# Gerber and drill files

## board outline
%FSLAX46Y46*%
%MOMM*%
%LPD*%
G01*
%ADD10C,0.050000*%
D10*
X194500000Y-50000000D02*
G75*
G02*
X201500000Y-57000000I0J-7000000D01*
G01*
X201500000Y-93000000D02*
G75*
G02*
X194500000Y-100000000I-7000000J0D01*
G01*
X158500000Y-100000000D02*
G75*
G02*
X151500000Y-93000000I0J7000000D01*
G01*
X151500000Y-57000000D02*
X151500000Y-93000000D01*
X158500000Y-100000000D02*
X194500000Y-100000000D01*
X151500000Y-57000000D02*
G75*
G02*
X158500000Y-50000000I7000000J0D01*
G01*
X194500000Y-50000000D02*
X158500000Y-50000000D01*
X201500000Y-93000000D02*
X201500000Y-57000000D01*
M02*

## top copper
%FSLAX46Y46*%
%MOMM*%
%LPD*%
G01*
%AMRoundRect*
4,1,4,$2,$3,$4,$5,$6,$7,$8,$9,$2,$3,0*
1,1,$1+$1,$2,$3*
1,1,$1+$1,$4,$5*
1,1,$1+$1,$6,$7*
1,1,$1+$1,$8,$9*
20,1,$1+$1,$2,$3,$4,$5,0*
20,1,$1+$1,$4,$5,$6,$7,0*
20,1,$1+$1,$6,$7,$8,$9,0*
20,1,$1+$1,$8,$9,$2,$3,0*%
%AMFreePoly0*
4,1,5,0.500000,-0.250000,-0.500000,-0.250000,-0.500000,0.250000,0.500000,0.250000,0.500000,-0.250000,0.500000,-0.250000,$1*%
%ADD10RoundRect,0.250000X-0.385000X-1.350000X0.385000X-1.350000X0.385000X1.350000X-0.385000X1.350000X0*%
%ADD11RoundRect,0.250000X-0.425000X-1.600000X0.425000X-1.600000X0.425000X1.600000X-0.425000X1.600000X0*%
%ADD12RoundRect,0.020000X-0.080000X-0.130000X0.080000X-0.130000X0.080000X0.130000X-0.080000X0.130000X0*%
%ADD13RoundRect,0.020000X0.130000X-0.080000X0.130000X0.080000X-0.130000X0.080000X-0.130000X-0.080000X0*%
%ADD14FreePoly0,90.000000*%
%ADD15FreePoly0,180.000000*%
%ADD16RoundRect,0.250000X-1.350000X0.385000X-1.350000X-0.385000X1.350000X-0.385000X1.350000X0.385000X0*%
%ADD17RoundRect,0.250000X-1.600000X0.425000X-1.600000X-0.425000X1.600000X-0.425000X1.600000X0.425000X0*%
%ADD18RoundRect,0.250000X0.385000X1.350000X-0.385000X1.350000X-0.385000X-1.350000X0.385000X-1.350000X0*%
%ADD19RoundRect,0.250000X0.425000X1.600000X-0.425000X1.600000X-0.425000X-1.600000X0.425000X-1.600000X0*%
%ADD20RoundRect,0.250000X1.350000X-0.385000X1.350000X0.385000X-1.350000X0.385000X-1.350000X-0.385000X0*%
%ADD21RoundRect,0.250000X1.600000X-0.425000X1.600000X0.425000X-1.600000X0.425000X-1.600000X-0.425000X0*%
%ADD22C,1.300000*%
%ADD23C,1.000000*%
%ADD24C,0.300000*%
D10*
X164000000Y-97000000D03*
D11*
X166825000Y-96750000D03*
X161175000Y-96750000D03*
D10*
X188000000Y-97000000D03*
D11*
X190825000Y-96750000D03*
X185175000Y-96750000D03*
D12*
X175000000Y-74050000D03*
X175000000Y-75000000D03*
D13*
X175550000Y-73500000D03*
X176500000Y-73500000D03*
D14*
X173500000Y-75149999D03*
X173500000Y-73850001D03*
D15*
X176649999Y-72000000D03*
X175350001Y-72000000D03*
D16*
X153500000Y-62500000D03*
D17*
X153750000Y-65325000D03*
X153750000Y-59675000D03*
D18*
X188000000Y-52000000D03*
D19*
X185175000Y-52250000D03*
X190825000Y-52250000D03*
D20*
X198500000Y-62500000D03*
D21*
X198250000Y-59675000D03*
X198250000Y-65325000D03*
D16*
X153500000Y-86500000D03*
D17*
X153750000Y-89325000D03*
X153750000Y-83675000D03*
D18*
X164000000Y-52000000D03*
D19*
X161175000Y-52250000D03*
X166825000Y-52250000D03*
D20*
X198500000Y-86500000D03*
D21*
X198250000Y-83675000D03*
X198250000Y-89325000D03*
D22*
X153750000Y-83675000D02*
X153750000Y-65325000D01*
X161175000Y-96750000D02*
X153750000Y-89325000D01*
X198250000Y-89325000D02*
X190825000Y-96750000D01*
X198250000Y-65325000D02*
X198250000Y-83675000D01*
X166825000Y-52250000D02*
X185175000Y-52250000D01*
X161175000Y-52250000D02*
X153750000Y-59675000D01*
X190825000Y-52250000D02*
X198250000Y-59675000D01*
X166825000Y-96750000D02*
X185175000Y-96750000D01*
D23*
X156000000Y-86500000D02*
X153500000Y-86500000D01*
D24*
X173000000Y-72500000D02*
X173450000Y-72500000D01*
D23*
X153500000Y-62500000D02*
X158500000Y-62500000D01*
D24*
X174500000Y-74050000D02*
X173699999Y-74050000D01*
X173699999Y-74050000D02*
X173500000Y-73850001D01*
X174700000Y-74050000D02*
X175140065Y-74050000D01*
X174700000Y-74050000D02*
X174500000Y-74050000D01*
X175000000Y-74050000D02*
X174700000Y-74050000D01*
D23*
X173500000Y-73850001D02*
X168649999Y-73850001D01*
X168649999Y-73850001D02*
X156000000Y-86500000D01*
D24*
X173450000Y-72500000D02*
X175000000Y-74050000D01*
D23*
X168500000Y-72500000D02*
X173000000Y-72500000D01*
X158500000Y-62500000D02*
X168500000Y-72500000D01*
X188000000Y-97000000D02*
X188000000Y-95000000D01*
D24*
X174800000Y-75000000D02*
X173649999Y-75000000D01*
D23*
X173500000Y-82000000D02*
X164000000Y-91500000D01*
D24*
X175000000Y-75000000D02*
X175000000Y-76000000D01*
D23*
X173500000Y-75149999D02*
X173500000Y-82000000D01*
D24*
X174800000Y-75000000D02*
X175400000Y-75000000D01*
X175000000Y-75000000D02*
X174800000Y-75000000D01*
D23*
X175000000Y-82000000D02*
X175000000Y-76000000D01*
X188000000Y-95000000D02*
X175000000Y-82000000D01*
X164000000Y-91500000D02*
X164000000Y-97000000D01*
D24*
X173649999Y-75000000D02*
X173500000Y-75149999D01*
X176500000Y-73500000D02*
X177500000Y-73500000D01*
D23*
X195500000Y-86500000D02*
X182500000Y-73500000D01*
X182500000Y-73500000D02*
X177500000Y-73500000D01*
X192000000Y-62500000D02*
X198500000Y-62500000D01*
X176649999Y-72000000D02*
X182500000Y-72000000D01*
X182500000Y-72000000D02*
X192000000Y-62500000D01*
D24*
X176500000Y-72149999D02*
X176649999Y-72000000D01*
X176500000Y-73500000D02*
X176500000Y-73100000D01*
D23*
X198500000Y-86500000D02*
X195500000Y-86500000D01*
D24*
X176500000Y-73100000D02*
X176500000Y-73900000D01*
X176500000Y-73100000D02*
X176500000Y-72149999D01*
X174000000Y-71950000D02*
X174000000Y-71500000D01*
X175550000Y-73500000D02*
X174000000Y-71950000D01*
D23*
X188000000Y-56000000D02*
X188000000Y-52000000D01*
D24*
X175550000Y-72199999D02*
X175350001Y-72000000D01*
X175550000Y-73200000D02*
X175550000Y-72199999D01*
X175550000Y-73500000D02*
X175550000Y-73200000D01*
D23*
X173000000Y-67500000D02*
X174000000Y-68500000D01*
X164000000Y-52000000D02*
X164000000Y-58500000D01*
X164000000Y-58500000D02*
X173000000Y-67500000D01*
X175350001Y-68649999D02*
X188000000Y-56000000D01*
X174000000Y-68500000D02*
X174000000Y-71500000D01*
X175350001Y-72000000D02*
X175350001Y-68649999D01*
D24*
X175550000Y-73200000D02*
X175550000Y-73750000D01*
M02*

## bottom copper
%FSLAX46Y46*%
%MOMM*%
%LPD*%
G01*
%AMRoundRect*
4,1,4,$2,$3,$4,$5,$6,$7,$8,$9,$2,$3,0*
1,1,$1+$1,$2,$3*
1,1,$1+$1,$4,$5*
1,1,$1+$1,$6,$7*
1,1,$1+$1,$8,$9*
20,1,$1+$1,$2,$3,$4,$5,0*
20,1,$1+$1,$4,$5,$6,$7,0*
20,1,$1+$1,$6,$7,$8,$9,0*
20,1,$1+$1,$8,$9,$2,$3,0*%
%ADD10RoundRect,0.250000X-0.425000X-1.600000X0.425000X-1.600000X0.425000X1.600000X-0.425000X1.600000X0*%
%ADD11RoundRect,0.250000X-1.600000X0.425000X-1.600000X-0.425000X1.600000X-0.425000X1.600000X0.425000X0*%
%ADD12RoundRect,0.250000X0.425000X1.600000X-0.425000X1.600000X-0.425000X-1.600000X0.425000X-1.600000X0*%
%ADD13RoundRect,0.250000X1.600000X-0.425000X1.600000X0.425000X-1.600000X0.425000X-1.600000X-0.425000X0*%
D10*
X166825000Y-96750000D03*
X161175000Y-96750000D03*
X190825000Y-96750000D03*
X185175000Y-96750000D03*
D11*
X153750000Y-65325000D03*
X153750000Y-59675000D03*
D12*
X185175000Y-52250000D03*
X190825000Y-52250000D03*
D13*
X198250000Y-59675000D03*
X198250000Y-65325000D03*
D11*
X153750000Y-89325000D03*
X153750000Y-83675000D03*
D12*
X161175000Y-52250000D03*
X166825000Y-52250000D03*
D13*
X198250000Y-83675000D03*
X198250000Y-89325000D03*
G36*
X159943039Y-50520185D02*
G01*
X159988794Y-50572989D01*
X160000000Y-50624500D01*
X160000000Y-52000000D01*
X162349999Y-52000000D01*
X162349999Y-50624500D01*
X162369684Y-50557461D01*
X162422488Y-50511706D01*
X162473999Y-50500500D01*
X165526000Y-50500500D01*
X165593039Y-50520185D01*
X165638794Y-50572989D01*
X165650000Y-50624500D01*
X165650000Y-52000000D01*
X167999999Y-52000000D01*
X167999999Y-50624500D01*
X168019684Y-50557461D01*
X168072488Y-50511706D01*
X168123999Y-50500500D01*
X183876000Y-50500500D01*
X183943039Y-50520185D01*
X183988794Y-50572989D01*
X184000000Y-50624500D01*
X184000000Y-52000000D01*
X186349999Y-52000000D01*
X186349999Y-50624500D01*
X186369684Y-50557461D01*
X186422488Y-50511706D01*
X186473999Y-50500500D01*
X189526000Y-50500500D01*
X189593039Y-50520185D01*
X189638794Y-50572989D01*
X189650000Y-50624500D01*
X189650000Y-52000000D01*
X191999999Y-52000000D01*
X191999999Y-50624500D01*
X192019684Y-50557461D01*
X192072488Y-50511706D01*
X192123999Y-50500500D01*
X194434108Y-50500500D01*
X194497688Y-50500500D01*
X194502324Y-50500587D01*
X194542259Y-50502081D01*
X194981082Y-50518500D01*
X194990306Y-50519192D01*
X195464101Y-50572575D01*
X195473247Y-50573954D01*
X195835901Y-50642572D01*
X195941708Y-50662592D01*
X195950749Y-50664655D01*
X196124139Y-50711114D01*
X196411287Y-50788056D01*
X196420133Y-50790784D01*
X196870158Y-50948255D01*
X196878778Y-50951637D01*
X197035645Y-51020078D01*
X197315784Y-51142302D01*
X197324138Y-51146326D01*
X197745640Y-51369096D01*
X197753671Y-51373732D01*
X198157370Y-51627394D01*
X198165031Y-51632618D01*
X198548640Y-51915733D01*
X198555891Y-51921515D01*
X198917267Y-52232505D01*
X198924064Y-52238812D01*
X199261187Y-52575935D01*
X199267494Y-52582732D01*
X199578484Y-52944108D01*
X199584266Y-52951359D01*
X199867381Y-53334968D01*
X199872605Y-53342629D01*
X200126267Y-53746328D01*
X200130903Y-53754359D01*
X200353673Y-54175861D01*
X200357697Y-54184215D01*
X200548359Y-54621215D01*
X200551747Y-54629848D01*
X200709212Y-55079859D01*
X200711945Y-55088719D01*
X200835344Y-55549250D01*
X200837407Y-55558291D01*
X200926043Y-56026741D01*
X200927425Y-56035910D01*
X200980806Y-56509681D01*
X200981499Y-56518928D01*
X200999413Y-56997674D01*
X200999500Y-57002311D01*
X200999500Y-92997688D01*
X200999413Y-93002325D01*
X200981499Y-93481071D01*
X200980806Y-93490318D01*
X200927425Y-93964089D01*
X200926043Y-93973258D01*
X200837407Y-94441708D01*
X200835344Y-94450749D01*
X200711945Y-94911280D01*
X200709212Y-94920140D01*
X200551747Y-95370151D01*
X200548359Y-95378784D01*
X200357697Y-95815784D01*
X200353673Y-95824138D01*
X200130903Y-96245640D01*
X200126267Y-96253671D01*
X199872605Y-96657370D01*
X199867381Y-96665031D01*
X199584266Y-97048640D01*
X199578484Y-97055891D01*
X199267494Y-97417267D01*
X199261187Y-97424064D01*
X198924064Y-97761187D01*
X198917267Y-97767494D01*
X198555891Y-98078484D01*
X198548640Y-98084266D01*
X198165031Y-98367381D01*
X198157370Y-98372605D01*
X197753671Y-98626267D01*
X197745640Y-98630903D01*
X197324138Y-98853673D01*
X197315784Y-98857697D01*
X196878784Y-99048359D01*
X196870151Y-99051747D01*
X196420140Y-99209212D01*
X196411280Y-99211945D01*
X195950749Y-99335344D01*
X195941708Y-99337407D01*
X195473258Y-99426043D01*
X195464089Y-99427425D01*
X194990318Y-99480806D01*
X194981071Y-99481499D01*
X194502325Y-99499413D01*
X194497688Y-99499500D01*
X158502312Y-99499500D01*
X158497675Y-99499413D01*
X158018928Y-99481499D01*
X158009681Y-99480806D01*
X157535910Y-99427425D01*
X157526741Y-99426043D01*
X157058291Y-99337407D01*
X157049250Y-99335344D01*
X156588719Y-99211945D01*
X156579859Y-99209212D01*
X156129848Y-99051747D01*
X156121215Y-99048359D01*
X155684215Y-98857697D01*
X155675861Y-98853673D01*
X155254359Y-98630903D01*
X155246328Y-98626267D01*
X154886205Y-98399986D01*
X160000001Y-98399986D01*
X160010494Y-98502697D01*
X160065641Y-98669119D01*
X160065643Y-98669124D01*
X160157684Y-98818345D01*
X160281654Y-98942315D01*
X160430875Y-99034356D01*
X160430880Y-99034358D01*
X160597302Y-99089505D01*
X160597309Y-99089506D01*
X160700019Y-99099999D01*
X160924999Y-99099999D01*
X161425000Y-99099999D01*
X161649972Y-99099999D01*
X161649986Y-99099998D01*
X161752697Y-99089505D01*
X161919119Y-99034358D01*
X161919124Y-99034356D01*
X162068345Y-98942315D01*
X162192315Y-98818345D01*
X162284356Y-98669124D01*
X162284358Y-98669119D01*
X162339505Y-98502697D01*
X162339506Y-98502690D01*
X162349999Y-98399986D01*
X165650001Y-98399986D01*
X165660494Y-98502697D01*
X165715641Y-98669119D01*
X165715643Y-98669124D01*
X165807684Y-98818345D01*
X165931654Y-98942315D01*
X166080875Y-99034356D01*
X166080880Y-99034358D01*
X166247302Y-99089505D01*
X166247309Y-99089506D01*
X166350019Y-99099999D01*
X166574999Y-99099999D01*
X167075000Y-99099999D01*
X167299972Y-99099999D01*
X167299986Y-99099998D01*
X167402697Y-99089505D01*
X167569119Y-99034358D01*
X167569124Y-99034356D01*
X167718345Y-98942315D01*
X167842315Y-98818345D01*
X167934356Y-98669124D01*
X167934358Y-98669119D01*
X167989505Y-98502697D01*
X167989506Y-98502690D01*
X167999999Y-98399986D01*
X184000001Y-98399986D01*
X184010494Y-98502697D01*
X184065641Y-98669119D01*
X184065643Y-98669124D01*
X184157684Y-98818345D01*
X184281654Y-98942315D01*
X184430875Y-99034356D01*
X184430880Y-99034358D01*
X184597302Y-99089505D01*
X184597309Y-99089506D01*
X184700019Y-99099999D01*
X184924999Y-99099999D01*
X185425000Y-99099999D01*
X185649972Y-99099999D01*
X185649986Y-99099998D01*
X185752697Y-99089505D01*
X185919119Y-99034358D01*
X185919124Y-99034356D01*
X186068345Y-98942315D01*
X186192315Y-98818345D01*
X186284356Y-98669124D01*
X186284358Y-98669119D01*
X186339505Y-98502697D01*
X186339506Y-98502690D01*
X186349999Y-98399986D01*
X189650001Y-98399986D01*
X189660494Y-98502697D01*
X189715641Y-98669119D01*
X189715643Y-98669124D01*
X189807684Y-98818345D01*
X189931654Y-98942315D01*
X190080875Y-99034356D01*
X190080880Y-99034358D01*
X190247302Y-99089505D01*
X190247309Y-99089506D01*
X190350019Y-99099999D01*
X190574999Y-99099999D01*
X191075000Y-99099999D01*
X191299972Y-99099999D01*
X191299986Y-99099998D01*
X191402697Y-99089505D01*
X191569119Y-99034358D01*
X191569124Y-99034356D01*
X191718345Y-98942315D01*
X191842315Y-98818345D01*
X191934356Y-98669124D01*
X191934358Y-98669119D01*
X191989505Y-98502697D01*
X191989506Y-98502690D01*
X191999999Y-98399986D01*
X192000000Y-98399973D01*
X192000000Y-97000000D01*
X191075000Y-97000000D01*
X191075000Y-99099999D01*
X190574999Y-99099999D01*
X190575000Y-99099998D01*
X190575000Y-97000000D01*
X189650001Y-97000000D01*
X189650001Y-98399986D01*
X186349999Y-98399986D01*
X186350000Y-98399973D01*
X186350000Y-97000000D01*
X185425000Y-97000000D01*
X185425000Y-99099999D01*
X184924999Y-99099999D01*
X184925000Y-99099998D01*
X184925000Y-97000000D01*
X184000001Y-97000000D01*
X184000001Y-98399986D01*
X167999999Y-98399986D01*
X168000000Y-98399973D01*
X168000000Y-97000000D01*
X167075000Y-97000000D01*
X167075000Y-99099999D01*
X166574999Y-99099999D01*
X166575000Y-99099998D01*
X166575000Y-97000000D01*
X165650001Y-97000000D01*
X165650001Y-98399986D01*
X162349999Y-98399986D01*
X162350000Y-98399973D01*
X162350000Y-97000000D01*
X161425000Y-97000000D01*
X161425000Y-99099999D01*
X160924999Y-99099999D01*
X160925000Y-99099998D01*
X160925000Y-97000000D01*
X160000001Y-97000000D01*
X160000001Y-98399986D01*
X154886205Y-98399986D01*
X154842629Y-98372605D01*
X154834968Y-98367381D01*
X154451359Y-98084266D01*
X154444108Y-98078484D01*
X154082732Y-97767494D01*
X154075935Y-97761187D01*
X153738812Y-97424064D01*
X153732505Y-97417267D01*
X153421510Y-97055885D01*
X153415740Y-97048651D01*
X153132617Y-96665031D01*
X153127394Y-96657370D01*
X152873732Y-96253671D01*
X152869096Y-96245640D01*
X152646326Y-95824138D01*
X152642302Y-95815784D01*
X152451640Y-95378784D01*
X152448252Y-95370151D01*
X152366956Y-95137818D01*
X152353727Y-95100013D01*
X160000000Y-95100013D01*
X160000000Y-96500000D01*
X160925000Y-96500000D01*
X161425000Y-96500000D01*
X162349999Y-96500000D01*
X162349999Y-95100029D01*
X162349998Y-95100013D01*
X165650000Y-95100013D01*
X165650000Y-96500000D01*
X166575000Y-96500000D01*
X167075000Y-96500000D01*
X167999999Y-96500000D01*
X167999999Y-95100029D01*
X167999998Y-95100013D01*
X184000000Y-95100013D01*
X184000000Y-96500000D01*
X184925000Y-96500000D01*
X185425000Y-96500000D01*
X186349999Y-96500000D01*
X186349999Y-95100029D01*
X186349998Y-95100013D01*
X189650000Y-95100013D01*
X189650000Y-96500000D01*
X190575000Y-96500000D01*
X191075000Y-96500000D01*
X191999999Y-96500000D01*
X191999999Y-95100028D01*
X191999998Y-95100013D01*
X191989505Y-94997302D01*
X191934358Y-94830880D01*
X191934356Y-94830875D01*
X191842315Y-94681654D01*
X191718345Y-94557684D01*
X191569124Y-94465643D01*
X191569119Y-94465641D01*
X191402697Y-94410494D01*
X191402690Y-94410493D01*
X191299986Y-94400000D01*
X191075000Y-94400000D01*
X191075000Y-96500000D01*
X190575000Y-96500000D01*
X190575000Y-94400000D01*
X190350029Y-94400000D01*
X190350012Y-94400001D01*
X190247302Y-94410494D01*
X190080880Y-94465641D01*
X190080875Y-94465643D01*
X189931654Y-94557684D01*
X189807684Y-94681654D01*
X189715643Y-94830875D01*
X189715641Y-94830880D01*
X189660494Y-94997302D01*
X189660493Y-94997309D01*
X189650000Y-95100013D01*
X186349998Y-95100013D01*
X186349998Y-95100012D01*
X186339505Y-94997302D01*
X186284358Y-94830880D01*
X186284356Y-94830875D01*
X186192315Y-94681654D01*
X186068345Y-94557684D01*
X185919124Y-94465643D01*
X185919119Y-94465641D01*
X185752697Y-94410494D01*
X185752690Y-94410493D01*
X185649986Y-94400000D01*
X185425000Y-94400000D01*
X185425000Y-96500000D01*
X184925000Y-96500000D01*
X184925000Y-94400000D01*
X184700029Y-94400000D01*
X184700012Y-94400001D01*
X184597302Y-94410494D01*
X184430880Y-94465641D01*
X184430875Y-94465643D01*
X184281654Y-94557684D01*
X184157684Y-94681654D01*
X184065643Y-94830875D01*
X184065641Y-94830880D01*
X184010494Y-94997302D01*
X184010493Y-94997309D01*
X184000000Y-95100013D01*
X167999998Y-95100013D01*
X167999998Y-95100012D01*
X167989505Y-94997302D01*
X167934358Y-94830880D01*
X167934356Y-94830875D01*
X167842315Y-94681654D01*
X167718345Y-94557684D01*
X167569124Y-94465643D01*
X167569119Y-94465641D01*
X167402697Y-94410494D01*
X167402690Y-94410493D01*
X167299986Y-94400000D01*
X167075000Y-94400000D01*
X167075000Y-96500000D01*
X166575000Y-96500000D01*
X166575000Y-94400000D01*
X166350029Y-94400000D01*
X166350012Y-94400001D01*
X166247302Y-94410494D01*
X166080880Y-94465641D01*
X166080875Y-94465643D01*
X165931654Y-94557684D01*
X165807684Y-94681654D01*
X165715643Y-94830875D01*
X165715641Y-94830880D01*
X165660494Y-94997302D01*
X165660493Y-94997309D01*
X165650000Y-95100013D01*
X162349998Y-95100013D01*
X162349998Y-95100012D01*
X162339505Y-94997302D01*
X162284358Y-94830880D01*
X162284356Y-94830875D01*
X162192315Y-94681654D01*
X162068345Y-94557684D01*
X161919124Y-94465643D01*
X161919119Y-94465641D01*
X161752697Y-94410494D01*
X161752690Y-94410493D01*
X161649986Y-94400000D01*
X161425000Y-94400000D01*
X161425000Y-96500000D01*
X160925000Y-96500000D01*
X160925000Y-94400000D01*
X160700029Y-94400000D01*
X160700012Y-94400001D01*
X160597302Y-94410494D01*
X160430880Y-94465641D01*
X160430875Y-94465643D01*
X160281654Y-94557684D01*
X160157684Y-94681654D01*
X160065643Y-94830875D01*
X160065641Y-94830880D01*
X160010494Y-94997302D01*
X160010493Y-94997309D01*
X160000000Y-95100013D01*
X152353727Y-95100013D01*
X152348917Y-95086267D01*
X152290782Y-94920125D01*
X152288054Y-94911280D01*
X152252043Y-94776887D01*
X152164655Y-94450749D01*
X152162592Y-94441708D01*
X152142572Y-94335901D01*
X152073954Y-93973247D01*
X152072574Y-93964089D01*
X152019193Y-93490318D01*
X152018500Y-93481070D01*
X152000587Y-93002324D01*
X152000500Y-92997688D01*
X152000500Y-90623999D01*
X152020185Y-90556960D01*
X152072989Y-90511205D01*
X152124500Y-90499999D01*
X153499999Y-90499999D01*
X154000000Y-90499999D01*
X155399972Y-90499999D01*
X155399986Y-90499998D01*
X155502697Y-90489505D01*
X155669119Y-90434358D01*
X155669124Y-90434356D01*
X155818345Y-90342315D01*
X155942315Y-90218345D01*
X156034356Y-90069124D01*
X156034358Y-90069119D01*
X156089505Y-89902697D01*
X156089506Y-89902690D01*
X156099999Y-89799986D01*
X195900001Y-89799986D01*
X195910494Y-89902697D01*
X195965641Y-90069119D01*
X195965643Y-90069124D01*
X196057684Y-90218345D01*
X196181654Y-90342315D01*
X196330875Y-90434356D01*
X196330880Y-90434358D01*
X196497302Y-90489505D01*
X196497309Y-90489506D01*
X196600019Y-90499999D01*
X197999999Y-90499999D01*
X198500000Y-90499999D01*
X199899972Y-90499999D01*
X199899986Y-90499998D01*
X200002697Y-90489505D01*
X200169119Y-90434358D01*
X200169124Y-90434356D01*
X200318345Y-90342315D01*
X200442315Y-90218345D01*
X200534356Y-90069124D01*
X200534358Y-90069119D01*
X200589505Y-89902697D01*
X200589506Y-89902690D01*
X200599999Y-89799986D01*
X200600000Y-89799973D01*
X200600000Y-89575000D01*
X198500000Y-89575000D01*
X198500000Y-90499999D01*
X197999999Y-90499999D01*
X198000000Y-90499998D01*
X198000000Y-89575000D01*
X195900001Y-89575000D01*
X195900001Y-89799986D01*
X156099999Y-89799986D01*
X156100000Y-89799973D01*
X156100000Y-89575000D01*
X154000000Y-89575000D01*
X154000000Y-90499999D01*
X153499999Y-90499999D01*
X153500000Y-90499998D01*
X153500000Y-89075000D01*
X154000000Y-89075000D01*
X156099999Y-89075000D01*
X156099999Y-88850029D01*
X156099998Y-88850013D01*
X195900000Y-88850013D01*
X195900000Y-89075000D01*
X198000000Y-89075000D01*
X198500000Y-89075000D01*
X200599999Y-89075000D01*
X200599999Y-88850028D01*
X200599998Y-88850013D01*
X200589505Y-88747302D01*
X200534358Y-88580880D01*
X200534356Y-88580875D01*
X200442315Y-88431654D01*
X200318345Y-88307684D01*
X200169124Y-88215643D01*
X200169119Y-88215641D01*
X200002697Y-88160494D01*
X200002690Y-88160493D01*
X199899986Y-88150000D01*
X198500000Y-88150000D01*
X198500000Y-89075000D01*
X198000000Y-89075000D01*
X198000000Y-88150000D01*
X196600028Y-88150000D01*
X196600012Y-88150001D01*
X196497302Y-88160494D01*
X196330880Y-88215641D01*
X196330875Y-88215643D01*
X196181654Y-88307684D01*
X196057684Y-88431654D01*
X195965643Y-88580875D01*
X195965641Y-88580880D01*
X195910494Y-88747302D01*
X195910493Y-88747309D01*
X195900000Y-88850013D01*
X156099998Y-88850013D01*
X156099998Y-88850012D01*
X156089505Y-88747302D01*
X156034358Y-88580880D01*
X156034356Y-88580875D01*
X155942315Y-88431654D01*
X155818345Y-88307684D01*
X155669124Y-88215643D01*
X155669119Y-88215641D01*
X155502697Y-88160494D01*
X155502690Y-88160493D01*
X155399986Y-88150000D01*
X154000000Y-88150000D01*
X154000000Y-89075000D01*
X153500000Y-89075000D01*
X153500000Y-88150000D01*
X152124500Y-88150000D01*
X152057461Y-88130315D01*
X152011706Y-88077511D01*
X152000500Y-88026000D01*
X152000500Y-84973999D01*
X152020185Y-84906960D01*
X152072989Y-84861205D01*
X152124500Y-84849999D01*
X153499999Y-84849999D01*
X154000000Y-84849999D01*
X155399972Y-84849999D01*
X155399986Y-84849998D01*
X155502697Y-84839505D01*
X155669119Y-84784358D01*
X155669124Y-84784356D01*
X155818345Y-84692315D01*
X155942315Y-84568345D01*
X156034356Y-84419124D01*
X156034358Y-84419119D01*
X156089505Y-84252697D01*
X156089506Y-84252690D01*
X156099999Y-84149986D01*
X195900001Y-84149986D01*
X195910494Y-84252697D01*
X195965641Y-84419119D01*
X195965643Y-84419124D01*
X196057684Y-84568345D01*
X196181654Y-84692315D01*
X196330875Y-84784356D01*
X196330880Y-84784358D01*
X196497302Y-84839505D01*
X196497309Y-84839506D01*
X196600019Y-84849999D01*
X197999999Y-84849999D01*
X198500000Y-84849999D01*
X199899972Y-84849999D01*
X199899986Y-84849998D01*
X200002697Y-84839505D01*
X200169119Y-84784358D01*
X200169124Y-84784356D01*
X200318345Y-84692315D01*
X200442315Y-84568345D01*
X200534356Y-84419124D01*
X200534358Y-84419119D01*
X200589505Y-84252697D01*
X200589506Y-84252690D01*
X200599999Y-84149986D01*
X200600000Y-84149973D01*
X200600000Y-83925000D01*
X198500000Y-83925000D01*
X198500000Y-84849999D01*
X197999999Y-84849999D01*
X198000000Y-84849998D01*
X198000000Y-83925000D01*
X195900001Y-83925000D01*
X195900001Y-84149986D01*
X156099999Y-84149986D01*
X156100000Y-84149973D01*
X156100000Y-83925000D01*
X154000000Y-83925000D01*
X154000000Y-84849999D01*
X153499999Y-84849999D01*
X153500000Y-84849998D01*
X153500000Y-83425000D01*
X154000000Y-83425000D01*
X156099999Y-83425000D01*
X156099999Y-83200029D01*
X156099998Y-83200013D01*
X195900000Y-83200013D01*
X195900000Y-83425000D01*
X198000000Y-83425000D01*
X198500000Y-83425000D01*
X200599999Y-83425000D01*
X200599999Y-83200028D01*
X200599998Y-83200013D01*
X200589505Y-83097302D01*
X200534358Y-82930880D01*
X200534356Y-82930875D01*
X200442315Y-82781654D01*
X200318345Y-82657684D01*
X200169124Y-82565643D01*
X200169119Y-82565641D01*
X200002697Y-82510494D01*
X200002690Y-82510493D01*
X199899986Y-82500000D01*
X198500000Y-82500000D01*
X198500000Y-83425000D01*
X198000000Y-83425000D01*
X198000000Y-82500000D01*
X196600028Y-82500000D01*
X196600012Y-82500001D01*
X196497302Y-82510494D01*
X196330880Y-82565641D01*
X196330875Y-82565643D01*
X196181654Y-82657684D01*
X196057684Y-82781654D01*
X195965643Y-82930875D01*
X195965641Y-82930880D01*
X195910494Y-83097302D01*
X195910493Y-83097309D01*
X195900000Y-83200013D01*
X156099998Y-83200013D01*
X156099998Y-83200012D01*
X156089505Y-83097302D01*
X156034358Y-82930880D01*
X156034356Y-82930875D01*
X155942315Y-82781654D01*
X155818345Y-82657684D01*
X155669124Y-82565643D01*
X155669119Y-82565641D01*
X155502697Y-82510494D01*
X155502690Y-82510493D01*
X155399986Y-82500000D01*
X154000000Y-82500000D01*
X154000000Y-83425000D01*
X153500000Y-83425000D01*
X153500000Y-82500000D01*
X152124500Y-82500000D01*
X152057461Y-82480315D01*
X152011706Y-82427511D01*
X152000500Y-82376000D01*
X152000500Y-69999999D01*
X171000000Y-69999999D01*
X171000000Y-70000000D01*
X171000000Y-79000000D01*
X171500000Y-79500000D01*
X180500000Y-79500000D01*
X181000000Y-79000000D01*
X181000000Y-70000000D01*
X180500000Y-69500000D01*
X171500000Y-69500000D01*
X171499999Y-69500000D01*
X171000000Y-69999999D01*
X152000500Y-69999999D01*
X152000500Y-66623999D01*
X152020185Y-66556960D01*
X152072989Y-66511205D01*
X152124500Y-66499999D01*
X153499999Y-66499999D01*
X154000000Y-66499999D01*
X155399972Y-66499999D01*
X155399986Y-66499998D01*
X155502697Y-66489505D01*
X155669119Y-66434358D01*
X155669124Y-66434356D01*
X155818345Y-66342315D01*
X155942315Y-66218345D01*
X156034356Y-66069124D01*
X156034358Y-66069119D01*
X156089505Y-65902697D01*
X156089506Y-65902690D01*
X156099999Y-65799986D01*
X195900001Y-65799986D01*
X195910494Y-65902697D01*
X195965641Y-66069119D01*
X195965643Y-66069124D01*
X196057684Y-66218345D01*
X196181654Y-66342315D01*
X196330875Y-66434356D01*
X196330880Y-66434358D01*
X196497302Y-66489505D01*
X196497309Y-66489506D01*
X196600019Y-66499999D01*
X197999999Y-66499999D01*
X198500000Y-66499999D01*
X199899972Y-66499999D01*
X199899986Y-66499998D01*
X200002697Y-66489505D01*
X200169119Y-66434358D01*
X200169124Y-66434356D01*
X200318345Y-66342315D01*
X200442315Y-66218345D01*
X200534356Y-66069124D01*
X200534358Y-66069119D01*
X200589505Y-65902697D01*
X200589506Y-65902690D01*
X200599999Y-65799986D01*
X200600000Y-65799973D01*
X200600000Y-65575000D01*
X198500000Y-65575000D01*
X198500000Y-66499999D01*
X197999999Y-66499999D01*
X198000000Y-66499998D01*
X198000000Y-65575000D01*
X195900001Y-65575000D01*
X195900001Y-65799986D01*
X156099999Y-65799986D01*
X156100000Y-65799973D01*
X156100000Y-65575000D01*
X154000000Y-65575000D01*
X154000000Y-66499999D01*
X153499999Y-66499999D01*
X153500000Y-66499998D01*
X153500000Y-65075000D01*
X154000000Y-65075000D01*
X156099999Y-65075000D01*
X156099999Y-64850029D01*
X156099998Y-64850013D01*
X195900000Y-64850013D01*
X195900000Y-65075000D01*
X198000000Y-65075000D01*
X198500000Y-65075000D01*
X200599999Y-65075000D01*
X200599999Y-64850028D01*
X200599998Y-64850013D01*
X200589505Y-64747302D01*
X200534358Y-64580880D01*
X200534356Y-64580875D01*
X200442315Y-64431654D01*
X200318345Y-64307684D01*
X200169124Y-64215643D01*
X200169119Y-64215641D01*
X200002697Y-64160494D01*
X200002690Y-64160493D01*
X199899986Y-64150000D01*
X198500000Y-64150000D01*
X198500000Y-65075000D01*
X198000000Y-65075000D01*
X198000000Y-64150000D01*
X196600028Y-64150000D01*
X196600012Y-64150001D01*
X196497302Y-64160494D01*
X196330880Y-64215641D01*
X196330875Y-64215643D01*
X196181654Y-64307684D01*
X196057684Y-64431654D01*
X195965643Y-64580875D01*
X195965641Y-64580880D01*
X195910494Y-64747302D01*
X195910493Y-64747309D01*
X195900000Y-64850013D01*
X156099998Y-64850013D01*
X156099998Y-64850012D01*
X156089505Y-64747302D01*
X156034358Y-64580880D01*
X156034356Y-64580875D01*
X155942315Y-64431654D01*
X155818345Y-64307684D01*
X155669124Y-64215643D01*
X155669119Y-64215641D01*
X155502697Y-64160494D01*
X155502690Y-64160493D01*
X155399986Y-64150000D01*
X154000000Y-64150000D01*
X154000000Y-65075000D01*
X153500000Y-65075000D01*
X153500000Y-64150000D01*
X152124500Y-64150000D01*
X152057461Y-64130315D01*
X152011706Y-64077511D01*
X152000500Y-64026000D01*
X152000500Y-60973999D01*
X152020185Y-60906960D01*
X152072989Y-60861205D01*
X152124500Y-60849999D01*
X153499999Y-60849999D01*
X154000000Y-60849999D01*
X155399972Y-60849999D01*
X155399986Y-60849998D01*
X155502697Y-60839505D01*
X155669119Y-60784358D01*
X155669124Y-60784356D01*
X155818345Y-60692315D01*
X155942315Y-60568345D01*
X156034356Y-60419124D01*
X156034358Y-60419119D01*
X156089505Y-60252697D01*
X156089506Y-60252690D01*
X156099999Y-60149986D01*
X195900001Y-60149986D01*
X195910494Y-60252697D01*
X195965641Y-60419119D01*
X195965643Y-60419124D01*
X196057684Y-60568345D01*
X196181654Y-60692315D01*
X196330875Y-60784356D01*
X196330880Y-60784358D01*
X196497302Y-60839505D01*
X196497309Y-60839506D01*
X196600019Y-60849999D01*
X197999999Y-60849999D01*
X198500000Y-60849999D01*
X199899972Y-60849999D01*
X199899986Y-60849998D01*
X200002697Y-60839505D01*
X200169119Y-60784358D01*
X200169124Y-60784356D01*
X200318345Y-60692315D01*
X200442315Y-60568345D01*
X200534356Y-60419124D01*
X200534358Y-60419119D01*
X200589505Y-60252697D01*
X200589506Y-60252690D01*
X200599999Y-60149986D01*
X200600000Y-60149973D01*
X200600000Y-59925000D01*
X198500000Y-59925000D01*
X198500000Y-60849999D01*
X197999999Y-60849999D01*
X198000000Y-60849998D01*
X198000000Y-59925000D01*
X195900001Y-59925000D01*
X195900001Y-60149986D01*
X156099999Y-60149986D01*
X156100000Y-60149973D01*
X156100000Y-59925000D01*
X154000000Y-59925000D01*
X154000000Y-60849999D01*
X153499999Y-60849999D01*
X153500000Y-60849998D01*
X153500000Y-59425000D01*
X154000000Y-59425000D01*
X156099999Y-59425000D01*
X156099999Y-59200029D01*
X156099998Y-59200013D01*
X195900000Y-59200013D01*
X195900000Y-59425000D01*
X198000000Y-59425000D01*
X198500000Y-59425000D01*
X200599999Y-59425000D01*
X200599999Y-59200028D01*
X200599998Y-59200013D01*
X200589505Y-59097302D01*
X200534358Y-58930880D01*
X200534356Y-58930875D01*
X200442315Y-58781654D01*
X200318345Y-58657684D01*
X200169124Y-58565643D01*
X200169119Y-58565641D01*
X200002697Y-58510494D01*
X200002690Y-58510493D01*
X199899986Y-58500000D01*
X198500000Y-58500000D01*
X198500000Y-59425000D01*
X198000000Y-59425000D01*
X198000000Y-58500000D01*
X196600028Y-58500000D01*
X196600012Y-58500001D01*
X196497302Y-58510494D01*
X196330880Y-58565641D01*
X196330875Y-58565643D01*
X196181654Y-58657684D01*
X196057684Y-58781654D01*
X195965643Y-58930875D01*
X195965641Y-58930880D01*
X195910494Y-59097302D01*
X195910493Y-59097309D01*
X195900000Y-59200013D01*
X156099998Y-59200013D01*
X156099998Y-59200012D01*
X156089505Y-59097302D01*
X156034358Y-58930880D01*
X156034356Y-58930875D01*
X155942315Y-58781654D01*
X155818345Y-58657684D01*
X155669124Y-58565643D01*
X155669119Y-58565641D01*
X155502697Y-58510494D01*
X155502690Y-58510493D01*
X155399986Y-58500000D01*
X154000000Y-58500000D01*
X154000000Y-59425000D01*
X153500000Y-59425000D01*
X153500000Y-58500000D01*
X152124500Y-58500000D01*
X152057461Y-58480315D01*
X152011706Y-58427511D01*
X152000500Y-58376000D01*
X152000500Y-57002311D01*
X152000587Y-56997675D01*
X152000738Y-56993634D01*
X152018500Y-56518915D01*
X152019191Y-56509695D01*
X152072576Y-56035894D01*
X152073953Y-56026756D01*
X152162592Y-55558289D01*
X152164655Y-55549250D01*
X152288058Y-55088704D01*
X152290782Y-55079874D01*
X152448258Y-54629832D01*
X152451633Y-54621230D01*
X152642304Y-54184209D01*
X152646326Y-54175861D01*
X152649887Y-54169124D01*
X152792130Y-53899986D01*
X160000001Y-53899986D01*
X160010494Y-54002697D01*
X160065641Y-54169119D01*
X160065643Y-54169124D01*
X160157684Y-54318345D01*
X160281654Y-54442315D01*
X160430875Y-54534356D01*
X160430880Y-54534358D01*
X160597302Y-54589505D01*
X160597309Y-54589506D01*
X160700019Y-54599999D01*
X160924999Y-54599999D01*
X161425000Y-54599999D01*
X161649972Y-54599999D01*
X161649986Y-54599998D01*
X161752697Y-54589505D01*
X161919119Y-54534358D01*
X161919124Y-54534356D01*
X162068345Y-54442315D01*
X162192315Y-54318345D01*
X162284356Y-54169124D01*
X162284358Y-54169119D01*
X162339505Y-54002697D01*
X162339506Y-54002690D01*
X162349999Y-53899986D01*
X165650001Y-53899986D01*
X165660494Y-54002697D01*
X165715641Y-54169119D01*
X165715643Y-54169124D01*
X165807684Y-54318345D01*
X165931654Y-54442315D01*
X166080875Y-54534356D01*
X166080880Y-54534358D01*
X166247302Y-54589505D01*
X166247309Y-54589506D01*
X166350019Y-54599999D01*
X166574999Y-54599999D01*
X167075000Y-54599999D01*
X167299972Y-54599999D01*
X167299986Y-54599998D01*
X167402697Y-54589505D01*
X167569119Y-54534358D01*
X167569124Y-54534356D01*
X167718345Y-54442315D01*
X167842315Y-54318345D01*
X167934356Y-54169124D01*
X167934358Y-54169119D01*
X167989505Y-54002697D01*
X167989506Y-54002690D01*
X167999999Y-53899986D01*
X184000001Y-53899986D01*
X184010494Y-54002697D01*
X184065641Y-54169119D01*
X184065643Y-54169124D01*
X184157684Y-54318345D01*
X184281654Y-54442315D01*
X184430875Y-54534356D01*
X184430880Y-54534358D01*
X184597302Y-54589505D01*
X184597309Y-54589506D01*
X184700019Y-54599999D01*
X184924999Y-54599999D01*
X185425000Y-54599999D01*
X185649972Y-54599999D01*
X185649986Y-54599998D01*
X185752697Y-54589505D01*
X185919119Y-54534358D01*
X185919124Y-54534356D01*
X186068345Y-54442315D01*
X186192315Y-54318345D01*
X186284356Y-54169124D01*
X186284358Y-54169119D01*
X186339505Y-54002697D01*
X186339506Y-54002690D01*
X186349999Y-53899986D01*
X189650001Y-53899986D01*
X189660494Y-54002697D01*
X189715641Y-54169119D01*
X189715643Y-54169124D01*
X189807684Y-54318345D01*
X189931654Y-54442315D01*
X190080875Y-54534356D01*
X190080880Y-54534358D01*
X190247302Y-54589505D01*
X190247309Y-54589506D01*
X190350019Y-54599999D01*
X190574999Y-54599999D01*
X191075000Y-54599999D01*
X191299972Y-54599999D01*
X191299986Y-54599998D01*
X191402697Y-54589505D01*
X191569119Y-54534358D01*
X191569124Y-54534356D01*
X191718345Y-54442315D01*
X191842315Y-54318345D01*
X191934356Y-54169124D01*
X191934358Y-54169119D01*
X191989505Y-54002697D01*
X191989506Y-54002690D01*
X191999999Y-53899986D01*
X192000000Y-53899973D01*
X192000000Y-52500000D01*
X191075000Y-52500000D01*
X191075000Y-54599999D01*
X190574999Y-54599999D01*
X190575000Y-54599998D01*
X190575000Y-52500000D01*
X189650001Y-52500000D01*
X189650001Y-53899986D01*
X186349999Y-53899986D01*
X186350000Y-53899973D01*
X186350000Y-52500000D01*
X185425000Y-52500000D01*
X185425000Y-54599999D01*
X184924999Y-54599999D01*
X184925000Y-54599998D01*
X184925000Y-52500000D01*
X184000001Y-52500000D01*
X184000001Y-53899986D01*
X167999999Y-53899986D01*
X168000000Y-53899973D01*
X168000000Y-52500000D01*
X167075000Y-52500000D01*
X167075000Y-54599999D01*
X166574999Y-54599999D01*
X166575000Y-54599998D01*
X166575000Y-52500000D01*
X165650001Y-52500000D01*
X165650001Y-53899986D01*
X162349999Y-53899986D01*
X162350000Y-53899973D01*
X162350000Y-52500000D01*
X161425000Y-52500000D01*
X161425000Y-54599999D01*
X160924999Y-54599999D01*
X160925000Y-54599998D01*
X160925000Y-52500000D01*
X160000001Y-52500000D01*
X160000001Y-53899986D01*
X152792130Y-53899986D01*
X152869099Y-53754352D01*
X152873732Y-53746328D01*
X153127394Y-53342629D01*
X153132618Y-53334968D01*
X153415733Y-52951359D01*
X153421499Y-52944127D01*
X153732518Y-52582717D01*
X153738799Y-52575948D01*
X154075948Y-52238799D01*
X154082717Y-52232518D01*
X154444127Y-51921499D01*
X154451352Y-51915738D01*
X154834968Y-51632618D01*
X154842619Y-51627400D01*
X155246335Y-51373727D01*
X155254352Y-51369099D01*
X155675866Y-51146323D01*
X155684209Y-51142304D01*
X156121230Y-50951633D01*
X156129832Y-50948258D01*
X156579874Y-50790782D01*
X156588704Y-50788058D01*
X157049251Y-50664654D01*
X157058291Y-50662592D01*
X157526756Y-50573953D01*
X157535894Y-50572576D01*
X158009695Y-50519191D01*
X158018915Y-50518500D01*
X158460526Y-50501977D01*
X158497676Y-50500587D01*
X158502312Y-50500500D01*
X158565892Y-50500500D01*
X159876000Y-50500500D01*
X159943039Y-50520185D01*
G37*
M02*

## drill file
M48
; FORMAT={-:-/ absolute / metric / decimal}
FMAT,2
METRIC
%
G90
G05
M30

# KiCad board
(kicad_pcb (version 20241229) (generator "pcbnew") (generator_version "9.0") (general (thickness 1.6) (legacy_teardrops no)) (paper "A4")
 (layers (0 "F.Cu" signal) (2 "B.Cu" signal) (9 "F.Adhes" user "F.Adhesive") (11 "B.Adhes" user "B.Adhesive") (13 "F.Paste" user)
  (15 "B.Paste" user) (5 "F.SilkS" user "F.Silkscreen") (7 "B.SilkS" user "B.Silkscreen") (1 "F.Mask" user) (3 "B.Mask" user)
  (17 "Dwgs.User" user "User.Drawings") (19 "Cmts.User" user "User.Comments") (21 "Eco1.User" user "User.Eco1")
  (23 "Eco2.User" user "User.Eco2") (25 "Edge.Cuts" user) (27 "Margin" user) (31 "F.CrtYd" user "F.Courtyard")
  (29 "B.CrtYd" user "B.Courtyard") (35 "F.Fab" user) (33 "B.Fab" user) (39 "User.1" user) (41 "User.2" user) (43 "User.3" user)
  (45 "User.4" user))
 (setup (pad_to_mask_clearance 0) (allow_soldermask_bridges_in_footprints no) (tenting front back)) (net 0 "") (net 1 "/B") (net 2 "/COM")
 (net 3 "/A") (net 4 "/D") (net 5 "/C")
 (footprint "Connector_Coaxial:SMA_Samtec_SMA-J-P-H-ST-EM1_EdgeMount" (layer "F.Cu") (at 164 97 -90)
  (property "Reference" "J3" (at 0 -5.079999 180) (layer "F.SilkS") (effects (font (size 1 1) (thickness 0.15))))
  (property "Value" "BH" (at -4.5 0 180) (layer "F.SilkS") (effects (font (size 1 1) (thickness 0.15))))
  (pad "1" smd roundrect (at 0 0) (size 1.27 3.2) (layers "F.Cu" "F.Mask") (roundrect_rratio 0.1968503937) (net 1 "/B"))
  (pad "2" smd roundrect (at -0.25 -2.825) (size 1.35 3.7) (layers "F.Cu" "F.Mask") (roundrect_rratio 0.1851851852) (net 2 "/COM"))
  (pad "2" smd roundrect (at -0.25 -2.825) (size 1.35 3.7) (layers "B.Cu" "B.Mask") (roundrect_rratio 0.1851851852) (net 2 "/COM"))
  (pad "2" smd roundrect (at -0.25 2.825) (size 1.35 3.7) (layers "F.Cu" "F.Mask") (roundrect_rratio 0.1851851852) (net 2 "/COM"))
  (pad "2" smd roundrect (at -0.25 2.825) (size 1.35 3.7) (layers "B.Cu" "B.Mask") (roundrect_rratio 0.1851851852) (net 2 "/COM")))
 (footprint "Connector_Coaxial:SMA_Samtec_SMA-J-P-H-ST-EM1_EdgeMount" (layer "F.Cu") (at 188 97 -90)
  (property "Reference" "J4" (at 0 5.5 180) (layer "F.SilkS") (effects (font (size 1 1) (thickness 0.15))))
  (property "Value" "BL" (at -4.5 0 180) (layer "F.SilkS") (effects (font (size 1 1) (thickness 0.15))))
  (pad "1" smd roundrect (at 0 0) (size 1.27 3.2) (layers "F.Cu" "F.Mask") (roundrect_rratio 0.1968503937) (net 1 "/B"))
  (pad "2" smd roundrect (at -0.25 -2.825) (size 1.35 3.7) (layers "F.Cu" "F.Mask") (roundrect_rratio 0.1851851852) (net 2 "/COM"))
  (pad "2" smd roundrect (at -0.25 -2.825) (size 1.35 3.7) (layers "B.Cu" "B.Mask") (roundrect_rratio 0.1851851852) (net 2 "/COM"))
  (pad "2" smd roundrect (at -0.25 2.825) (size 1.35 3.7) (layers "F.Cu" "F.Mask") (roundrect_rratio 0.1851851852) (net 2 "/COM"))
  (pad "2" smd roundrect (at -0.25 2.825) (size 1.35 3.7) (layers "B.Cu" "B.Mask") (roundrect_rratio 0.1851851852) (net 2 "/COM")))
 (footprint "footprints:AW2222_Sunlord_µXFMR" (layer "F.Cu") (at 174.9 73.4)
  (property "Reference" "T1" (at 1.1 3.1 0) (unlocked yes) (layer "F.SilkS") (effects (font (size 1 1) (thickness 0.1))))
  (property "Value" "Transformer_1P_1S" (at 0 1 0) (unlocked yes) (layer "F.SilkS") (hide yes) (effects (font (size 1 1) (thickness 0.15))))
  (pad "1" smd roundrect (at 0.1 0.65) (size 0.2 0.3) (layers "F.Cu" "F.Mask" "F.Paste") (roundrect_rratio 0.1) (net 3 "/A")
   (thermal_bridge_angle 45))
  (pad "2" smd roundrect (at 0.1 1.6) (size 0.2 0.3) (layers "F.Cu" "F.Mask" "F.Paste") (roundrect_rratio 0.1) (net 1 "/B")
   (thermal_bridge_angle 45))
  (pad "3" smd roundrect (at 0.65 0.1 90) (size 0.2 0.3) (layers "F.Cu" "F.Mask" "F.Paste") (roundrect_rratio 0.1) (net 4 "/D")
   (thermal_bridge_angle 45))
  (pad "4" smd roundrect (at 1.6 0.1 90) (size 0.2 0.3) (layers "F.Cu" "F.Mask" "F.Paste") (roundrect_rratio 0.1) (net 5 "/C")
   (thermal_bridge_angle 45)))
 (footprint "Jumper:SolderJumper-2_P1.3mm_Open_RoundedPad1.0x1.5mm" (layer "F.Cu") (at 173.5 74.5 90)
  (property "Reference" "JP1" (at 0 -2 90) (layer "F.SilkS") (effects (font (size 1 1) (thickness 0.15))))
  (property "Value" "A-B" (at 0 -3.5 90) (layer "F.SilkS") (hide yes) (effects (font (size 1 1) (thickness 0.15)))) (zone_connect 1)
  (pad "1" smd custom (at -0.649999 0 90) (size 1 0.5) (layers "F.Cu" "F.Mask") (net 1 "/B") (zone_connect 2) (thermal_bridge_angle 45)
   (options (clearance outline) (anchor rect)) (primitives))
  (pad "2" smd custom (at 0.649999 0 90) (size 1 0.5) (layers "F.Cu" "F.Mask") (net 3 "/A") (zone_connect 2) (thermal_bridge_angle 45)
   (options (clearance outline) (anchor rect)) (primitives)))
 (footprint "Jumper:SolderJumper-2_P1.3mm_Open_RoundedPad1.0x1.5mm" (layer "F.Cu") (at 176 72 180)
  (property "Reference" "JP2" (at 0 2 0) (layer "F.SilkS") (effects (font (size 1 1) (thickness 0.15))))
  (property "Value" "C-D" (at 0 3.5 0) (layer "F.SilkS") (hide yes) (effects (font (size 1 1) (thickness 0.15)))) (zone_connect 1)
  (pad "1" smd custom (at -0.649999 0 180) (size 1 0.5) (layers "F.Cu" "F.Mask") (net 5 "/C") (zone_connect 2) (thermal_bridge_angle 45)
   (options (clearance outline) (anchor rect)) (primitives))
  (pad "2" smd custom (at 0.649999 0 180) (size 1 0.5) (layers "F.Cu" "F.Mask") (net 4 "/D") (zone_connect 2) (thermal_bridge_angle 45)
   (options (clearance outline) (anchor rect)) (primitives)))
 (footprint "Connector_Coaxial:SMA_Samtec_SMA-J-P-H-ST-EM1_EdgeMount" (layer "F.Cu") (at 153.5 62.5 180)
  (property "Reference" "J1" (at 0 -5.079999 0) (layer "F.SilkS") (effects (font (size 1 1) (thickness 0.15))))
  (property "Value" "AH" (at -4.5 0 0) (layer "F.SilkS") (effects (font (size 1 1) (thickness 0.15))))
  (pad "1" smd roundrect (at 0 0 270) (size 1.27 3.2) (layers "F.Cu" "F.Mask") (roundrect_rratio 0.1968503937) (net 3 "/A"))
  (pad "2" smd roundrect (at -0.25 -2.825 270) (size 1.35 3.7) (layers "F.Cu" "F.Mask") (roundrect_rratio 0.1851851852) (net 2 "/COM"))
  (pad "2" smd roundrect (at -0.25 -2.825 270) (size 1.35 3.7) (layers "B.Cu" "B.Mask") (roundrect_rratio 0.1851851852) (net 2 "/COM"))
  (pad "2" smd roundrect (at -0.25 2.825 270) (size 1.35 3.7) (layers "F.Cu" "F.Mask") (roundrect_rratio 0.1851851852) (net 2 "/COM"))
  (pad "2" smd roundrect (at -0.25 2.825 270) (size 1.35 3.7) (layers "B.Cu" "B.Mask") (roundrect_rratio 0.1851851852) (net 2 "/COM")))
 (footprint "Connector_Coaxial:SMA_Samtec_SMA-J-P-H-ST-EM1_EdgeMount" (layer "F.Cu") (at 188 52 90)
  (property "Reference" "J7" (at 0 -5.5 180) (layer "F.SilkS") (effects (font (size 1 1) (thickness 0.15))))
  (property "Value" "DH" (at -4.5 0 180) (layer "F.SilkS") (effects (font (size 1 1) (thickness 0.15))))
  (pad "1" smd roundrect (at 0 0 180) (size 1.27 3.2) (layers "F.Cu" "F.Mask") (roundrect_rratio 0.1968503937) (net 4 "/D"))
  (pad "2" smd roundrect (at -0.25 -2.825 180) (size 1.35 3.7) (layers "F.Cu" "F.Mask") (roundrect_rratio 0.1851851852) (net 2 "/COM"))
  (pad "2" smd roundrect (at -0.25 -2.825 180) (size 1.35 3.7) (layers "B.Cu" "B.Mask") (roundrect_rratio 0.1851851852) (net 2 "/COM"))
  (pad "2" smd roundrect (at -0.25 2.825 180) (size 1.35 3.7) (layers "F.Cu" "F.Mask") (roundrect_rratio 0.1851851852) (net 2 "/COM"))
  (pad "2" smd roundrect (at -0.25 2.825 180) (size 1.35 3.7) (layers "B.Cu" "B.Mask") (roundrect_rratio 0.1851851852) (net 2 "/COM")))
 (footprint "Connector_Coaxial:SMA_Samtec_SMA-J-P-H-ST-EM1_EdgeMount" (layer "F.Cu") (at 198.5 62.5)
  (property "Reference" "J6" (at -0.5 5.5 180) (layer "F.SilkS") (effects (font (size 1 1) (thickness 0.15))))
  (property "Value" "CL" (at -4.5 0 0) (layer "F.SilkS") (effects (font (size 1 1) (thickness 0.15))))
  (pad "1" smd roundrect (at 0 0 90) (size 1.27 3.2) (layers "F.Cu" "F.Mask") (roundrect_rratio 0.1968503937) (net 5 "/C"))
  (pad "2" smd roundrect (at -0.25 -2.825 90) (size 1.35 3.7) (layers "F.Cu" "F.Mask") (roundrect_rratio 0.1851851852) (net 2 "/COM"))
  (pad "2" smd roundrect (at -0.25 -2.825 90) (size 1.35 3.7) (layers "B.Cu" "B.Mask") (roundrect_rratio 0.1851851852) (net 2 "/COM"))
  (pad "2" smd roundrect (at -0.25 2.825 90) (size 1.35 3.7) (layers "F.Cu" "F.Mask") (roundrect_rratio 0.1851851852) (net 2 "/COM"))
  (pad "2" smd roundrect (at -0.25 2.825 90) (size 1.35 3.7) (layers "B.Cu" "B.Mask") (roundrect_rratio 0.1851851852) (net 2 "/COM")))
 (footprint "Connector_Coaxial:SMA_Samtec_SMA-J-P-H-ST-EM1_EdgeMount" (layer "F.Cu") (at 153.5 86.5 180)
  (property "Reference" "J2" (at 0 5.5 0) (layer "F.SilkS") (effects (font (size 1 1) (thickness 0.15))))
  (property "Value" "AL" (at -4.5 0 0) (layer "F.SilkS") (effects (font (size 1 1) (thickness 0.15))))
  (pad "1" smd roundrect (at 0 0 270) (size 1.27 3.2) (layers "F.Cu" "F.Mask") (roundrect_rratio 0.1968503937) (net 3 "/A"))
  (pad "2" smd roundrect (at -0.25 -2.825 270) (size 1.35 3.7) (layers "F.Cu" "F.Mask") (roundrect_rratio 0.1851851852) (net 2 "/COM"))
  (pad "2" smd roundrect (at -0.25 -2.825 270) (size 1.35 3.7) (layers "B.Cu" "B.Mask") (roundrect_rratio 0.1851851852) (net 2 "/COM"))
  (pad "2" smd roundrect (at -0.25 2.825 270) (size 1.35 3.7) (layers "F.Cu" "F.Mask") (roundrect_rratio 0.1851851852) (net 2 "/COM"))
  (pad "2" smd roundrect (at -0.25 2.825 270) (size 1.35 3.7) (layers "B.Cu" "B.Mask") (roundrect_rratio 0.1851851852) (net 2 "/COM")))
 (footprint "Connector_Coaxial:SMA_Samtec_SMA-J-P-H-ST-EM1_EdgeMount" (layer "F.Cu") (at 164 52 90)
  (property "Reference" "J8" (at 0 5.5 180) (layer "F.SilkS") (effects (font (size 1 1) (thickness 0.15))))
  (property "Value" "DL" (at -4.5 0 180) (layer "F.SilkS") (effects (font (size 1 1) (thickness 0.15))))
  (pad "1" smd roundrect (at 0 0 180) (size 1.27 3.2) (layers "F.Cu" "F.Mask") (roundrect_rratio 0.1968503937) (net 4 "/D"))
  (pad "2" smd roundrect (at -0.25 -2.825 180) (size 1.35 3.7) (layers "F.Cu" "F.Mask") (roundrect_rratio 0.1851851852) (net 2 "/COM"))
  (pad "2" smd roundrect (at -0.25 -2.825 180) (size 1.35 3.7) (layers "B.Cu" "B.Mask") (roundrect_rratio 0.1851851852) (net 2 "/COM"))
  (pad "2" smd roundrect (at -0.25 2.825 180) (size 1.35 3.7) (layers "F.Cu" "F.Mask") (roundrect_rratio 0.1851851852) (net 2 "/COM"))
  (pad "2" smd roundrect (at -0.25 2.825 180) (size 1.35 3.7) (layers "B.Cu" "B.Mask") (roundrect_rratio 0.1851851852) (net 2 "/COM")))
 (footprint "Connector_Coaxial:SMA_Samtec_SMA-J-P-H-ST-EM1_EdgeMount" (layer "F.Cu") (at 198.5 86.5)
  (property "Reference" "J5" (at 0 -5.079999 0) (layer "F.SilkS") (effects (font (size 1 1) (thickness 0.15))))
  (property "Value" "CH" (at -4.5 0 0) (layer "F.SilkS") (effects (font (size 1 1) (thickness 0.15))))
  (pad "1" smd roundrect (at 0 0 90) (size 1.27 3.2) (layers "F.Cu" "F.Mask") (roundrect_rratio 0.1968503937) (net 5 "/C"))
  (pad "2" smd roundrect (at -0.25 -2.825 90) (size 1.35 3.7) (layers "F.Cu" "F.Mask") (roundrect_rratio 0.1851851852) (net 2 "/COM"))
  (pad "2" smd roundrect (at -0.25 -2.825 90) (size 1.35 3.7) (layers "B.Cu" "B.Mask") (roundrect_rratio 0.1851851852) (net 2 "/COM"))
  (pad "2" smd roundrect (at -0.25 2.825 90) (size 1.35 3.7) (layers "F.Cu" "F.Mask") (roundrect_rratio 0.1851851852) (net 2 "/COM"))
  (pad "2" smd roundrect (at -0.25 2.825 90) (size 1.35 3.7) (layers "B.Cu" "B.Mask") (roundrect_rratio 0.1851851852) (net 2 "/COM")))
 (gr_arc (start 194.5 50) (mid 199.449747 52.050253) (end 201.5 57) (stroke (width 0.05) (type default)) (layer "Edge.Cuts"))
 (gr_arc (start 201.5 93) (mid 199.449747 97.949747) (end 194.5 100) (stroke (width 0.05) (type default)) (layer "Edge.Cuts"))
 (gr_arc (start 158.5 100) (mid 153.550253 97.949747) (end 151.5 93) (stroke (width 0.05) (type default)) (layer "Edge.Cuts"))
 (gr_line (start 151.5 57) (end 151.5 93) (stroke (width 0.05) (type default)) (layer "Edge.Cuts"))
 (gr_line (start 158.5 100) (end 194.5 100) (stroke (width 0.05) (type default)) (layer "Edge.Cuts"))
 (gr_arc (start 151.5 57) (mid 153.550253 52.050253) (end 158.5 50) (stroke (width 0.05) (type default)) (layer "Edge.Cuts"))
 (gr_line (start 194.5 50) (end 158.5 50) (stroke (width 0.05) (type default)) (layer "Edge.Cuts"))
 (gr_line (start 201.5 93) (end 201.5 57) (stroke (width 0.05) (type default)) (layer "Edge.Cuts"))
 (segment (start 153.75 83.675) (end 153.75 65.325) (width 1.3) (layer "F.Cu") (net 2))
 (segment (start 161.175 96.75) (end 153.75 89.325) (width 1.3) (layer "F.Cu") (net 2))
 (segment (start 198.25 89.325) (end 190.825 96.75) (width 1.3) (layer "F.Cu") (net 2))
 (segment (start 198.25 65.325) (end 198.25 83.675) (width 1.3) (layer "F.Cu") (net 2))
 (segment (start 166.825 52.25) (end 185.175 52.25) (width 1.3) (layer "F.Cu") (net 2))
 (segment (start 161.175 52.25) (end 153.75 59.675) (width 1.3) (layer "F.Cu") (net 2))
 (segment (start 190.825 52.25) (end 198.25 59.675) (width 1.3) (layer "F.Cu") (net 2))
 (segment (start 166.825 96.75) (end 185.175 96.75) (width 1.3) (layer "F.Cu") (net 2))
 (segment (start 156 86.5) (end 153.5 86.5) (width 1) (layer "F.Cu") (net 3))
 (segment (start 173 72.5) (end 173.45 72.5) (width 0.3) (layer "F.Cu") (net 3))
 (segment (start 153.5 62.5) (end 158.5 62.5) (width 1) (layer "F.Cu") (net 3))
 (segment (start 174.5 74.05) (end 173.699999 74.05) (width 0.3) (layer "F.Cu") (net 3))
 (segment (start 173.699999 74.05) (end 173.5 73.850001) (width 0.3) (layer "F.Cu") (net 3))
 (segment (start 174.7 74.05) (end 175.140065 74.05) (width 0.3) (layer "F.Cu") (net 3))
 (segment (start 174.7 74.05) (end 174.5 74.05) (width 0.3) (layer "F.Cu") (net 3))
 (segment (start 175 74.05) (end 174.7 74.05) (width 0.3) (layer "F.Cu") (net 3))
 (segment (start 173.5 73.850001) (end 168.649999 73.850001) (width 1) (layer "F.Cu") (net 3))
 (segment (start 168.649999 73.850001) (end 156 86.5) (width 1) (layer "F.Cu") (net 3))
 (segment (start 173.45 72.5) (end 175 74.05) (width 0.3) (layer "F.Cu") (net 3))
 (segment (start 168.5 72.5) (end 173 72.5) (width 1) (layer "F.Cu") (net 3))
 (segment (start 158.5 62.5) (end 168.5 72.5) (width 1) (layer "F.Cu") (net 3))
 (segment (start 188 97) (end 188 95) (width 1) (layer "F.Cu") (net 1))
 (segment (start 174.8 75) (end 173.649999 75) (width 0.3) (layer "F.Cu") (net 1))
 (segment (start 173.5 82) (end 164 91.5) (width 1) (layer "F.Cu") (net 1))
 (segment (start 175 75) (end 175 76) (width 0.3) (layer "F.Cu") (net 1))
 (segment (start 173.5 75.149999) (end 173.5 82) (width 1) (layer "F.Cu") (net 1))
 (segment (start 174.8 75) (end 175.4 75) (width 0.3) (layer "F.Cu") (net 1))
 (segment (start 175 75) (end 174.8 75) (width 0.3) (layer "F.Cu") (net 1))
 (segment (start 175 82) (end 175 76) (width 1) (layer "F.Cu") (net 1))
 (segment (start 188 95) (end 175 82) (width 1) (layer "F.Cu") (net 1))
 (segment (start 164 91.5) (end 164 97) (width 1) (layer "F.Cu") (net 1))
 (segment (start 173.649999 75) (end 173.5 75.149999) (width 0.3) (layer "F.Cu") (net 1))
 (segment (start 176.5 73.5) (end 177.5 73.5) (width 0.3) (layer "F.Cu") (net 5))
 (segment (start 195.5 86.5) (end 182.5 73.5) (width 1) (layer "F.Cu") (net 5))
 (segment (start 182.5 73.5) (end 177.5 73.5) (width 1) (layer "F.Cu") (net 5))
 (segment (start 192 62.5) (end 198.5 62.5) (width 1) (layer "F.Cu") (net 5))
 (segment (start 176.649999 72) (end 182.5 72) (width 1) (layer "F.Cu") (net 5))
 (segment (start 182.5 72) (end 192 62.5) (width 1) (layer "F.Cu") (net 5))
 (segment (start 176.5 72.149999) (end 176.649999 72) (width 0.3) (layer "F.Cu") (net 5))
 (segment (start 176.5 73.5) (end 176.5 73.1) (width 0.3) (layer "F.Cu") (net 5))
 (segment (start 198.5 86.5) (end 195.5 86.5) (width 1) (layer "F.Cu") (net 5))
 (segment (start 176.5 73.1) (end 176.5 73.9) (width 0.3) (layer "F.Cu") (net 5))
 (segment (start 176.5 73.1) (end 176.5 72.149999) (width 0.3) (layer "F.Cu") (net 5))
 (segment (start 174 71.95) (end 174 71.5) (width 0.3) (layer "F.Cu") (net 4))
 (segment (start 175.55 73.5) (end 174 71.95) (width 0.3) (layer "F.Cu") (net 4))
 (segment (start 188 56) (end 188 52) (width 1) (layer "F.Cu") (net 4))
 (segment (start 175.55 72.199999) (end 175.350001 72) (width 0.3) (layer "F.Cu") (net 4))
 (segment (start 175.55 73.2) (end 175.55 72.199999) (width 0.3) (layer "F.Cu") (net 4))
 (segment (start 175.55 73.5) (end 175.55 73.2) (width 0.3) (layer "F.Cu") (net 4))
 (segment (start 173 67.5) (end 174 68.5) (width 1) (layer "F.Cu") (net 4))
 (segment (start 164 52) (end 164 58.5) (width 1) (layer "F.Cu") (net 4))
 (segment (start 164 58.5) (end 173 67.5) (width 1) (layer "F.Cu") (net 4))
 (segment (start 175.350001 68.649999) (end 188 56) (width 1) (layer "F.Cu") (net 4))
 (segment (start 174 68.5) (end 174 71.5) (width 1) (layer "F.Cu") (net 4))
 (segment (start 175.350001 72) (end 175.350001 68.649999) (width 1) (layer "F.Cu") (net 4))
 (segment (start 175.55 73.2) (end 175.55 73.75) (width 0.3) (layer "F.Cu") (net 4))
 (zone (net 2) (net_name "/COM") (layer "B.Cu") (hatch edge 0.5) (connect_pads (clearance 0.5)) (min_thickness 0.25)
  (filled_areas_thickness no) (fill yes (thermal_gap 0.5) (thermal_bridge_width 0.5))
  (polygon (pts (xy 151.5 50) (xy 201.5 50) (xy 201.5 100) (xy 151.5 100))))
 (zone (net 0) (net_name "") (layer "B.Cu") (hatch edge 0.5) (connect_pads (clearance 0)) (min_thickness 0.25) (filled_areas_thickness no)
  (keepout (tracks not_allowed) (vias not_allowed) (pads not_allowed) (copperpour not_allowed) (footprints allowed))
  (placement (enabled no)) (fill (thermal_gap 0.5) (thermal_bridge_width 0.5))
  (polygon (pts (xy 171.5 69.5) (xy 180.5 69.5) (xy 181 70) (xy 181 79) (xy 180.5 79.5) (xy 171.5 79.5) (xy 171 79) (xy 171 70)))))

